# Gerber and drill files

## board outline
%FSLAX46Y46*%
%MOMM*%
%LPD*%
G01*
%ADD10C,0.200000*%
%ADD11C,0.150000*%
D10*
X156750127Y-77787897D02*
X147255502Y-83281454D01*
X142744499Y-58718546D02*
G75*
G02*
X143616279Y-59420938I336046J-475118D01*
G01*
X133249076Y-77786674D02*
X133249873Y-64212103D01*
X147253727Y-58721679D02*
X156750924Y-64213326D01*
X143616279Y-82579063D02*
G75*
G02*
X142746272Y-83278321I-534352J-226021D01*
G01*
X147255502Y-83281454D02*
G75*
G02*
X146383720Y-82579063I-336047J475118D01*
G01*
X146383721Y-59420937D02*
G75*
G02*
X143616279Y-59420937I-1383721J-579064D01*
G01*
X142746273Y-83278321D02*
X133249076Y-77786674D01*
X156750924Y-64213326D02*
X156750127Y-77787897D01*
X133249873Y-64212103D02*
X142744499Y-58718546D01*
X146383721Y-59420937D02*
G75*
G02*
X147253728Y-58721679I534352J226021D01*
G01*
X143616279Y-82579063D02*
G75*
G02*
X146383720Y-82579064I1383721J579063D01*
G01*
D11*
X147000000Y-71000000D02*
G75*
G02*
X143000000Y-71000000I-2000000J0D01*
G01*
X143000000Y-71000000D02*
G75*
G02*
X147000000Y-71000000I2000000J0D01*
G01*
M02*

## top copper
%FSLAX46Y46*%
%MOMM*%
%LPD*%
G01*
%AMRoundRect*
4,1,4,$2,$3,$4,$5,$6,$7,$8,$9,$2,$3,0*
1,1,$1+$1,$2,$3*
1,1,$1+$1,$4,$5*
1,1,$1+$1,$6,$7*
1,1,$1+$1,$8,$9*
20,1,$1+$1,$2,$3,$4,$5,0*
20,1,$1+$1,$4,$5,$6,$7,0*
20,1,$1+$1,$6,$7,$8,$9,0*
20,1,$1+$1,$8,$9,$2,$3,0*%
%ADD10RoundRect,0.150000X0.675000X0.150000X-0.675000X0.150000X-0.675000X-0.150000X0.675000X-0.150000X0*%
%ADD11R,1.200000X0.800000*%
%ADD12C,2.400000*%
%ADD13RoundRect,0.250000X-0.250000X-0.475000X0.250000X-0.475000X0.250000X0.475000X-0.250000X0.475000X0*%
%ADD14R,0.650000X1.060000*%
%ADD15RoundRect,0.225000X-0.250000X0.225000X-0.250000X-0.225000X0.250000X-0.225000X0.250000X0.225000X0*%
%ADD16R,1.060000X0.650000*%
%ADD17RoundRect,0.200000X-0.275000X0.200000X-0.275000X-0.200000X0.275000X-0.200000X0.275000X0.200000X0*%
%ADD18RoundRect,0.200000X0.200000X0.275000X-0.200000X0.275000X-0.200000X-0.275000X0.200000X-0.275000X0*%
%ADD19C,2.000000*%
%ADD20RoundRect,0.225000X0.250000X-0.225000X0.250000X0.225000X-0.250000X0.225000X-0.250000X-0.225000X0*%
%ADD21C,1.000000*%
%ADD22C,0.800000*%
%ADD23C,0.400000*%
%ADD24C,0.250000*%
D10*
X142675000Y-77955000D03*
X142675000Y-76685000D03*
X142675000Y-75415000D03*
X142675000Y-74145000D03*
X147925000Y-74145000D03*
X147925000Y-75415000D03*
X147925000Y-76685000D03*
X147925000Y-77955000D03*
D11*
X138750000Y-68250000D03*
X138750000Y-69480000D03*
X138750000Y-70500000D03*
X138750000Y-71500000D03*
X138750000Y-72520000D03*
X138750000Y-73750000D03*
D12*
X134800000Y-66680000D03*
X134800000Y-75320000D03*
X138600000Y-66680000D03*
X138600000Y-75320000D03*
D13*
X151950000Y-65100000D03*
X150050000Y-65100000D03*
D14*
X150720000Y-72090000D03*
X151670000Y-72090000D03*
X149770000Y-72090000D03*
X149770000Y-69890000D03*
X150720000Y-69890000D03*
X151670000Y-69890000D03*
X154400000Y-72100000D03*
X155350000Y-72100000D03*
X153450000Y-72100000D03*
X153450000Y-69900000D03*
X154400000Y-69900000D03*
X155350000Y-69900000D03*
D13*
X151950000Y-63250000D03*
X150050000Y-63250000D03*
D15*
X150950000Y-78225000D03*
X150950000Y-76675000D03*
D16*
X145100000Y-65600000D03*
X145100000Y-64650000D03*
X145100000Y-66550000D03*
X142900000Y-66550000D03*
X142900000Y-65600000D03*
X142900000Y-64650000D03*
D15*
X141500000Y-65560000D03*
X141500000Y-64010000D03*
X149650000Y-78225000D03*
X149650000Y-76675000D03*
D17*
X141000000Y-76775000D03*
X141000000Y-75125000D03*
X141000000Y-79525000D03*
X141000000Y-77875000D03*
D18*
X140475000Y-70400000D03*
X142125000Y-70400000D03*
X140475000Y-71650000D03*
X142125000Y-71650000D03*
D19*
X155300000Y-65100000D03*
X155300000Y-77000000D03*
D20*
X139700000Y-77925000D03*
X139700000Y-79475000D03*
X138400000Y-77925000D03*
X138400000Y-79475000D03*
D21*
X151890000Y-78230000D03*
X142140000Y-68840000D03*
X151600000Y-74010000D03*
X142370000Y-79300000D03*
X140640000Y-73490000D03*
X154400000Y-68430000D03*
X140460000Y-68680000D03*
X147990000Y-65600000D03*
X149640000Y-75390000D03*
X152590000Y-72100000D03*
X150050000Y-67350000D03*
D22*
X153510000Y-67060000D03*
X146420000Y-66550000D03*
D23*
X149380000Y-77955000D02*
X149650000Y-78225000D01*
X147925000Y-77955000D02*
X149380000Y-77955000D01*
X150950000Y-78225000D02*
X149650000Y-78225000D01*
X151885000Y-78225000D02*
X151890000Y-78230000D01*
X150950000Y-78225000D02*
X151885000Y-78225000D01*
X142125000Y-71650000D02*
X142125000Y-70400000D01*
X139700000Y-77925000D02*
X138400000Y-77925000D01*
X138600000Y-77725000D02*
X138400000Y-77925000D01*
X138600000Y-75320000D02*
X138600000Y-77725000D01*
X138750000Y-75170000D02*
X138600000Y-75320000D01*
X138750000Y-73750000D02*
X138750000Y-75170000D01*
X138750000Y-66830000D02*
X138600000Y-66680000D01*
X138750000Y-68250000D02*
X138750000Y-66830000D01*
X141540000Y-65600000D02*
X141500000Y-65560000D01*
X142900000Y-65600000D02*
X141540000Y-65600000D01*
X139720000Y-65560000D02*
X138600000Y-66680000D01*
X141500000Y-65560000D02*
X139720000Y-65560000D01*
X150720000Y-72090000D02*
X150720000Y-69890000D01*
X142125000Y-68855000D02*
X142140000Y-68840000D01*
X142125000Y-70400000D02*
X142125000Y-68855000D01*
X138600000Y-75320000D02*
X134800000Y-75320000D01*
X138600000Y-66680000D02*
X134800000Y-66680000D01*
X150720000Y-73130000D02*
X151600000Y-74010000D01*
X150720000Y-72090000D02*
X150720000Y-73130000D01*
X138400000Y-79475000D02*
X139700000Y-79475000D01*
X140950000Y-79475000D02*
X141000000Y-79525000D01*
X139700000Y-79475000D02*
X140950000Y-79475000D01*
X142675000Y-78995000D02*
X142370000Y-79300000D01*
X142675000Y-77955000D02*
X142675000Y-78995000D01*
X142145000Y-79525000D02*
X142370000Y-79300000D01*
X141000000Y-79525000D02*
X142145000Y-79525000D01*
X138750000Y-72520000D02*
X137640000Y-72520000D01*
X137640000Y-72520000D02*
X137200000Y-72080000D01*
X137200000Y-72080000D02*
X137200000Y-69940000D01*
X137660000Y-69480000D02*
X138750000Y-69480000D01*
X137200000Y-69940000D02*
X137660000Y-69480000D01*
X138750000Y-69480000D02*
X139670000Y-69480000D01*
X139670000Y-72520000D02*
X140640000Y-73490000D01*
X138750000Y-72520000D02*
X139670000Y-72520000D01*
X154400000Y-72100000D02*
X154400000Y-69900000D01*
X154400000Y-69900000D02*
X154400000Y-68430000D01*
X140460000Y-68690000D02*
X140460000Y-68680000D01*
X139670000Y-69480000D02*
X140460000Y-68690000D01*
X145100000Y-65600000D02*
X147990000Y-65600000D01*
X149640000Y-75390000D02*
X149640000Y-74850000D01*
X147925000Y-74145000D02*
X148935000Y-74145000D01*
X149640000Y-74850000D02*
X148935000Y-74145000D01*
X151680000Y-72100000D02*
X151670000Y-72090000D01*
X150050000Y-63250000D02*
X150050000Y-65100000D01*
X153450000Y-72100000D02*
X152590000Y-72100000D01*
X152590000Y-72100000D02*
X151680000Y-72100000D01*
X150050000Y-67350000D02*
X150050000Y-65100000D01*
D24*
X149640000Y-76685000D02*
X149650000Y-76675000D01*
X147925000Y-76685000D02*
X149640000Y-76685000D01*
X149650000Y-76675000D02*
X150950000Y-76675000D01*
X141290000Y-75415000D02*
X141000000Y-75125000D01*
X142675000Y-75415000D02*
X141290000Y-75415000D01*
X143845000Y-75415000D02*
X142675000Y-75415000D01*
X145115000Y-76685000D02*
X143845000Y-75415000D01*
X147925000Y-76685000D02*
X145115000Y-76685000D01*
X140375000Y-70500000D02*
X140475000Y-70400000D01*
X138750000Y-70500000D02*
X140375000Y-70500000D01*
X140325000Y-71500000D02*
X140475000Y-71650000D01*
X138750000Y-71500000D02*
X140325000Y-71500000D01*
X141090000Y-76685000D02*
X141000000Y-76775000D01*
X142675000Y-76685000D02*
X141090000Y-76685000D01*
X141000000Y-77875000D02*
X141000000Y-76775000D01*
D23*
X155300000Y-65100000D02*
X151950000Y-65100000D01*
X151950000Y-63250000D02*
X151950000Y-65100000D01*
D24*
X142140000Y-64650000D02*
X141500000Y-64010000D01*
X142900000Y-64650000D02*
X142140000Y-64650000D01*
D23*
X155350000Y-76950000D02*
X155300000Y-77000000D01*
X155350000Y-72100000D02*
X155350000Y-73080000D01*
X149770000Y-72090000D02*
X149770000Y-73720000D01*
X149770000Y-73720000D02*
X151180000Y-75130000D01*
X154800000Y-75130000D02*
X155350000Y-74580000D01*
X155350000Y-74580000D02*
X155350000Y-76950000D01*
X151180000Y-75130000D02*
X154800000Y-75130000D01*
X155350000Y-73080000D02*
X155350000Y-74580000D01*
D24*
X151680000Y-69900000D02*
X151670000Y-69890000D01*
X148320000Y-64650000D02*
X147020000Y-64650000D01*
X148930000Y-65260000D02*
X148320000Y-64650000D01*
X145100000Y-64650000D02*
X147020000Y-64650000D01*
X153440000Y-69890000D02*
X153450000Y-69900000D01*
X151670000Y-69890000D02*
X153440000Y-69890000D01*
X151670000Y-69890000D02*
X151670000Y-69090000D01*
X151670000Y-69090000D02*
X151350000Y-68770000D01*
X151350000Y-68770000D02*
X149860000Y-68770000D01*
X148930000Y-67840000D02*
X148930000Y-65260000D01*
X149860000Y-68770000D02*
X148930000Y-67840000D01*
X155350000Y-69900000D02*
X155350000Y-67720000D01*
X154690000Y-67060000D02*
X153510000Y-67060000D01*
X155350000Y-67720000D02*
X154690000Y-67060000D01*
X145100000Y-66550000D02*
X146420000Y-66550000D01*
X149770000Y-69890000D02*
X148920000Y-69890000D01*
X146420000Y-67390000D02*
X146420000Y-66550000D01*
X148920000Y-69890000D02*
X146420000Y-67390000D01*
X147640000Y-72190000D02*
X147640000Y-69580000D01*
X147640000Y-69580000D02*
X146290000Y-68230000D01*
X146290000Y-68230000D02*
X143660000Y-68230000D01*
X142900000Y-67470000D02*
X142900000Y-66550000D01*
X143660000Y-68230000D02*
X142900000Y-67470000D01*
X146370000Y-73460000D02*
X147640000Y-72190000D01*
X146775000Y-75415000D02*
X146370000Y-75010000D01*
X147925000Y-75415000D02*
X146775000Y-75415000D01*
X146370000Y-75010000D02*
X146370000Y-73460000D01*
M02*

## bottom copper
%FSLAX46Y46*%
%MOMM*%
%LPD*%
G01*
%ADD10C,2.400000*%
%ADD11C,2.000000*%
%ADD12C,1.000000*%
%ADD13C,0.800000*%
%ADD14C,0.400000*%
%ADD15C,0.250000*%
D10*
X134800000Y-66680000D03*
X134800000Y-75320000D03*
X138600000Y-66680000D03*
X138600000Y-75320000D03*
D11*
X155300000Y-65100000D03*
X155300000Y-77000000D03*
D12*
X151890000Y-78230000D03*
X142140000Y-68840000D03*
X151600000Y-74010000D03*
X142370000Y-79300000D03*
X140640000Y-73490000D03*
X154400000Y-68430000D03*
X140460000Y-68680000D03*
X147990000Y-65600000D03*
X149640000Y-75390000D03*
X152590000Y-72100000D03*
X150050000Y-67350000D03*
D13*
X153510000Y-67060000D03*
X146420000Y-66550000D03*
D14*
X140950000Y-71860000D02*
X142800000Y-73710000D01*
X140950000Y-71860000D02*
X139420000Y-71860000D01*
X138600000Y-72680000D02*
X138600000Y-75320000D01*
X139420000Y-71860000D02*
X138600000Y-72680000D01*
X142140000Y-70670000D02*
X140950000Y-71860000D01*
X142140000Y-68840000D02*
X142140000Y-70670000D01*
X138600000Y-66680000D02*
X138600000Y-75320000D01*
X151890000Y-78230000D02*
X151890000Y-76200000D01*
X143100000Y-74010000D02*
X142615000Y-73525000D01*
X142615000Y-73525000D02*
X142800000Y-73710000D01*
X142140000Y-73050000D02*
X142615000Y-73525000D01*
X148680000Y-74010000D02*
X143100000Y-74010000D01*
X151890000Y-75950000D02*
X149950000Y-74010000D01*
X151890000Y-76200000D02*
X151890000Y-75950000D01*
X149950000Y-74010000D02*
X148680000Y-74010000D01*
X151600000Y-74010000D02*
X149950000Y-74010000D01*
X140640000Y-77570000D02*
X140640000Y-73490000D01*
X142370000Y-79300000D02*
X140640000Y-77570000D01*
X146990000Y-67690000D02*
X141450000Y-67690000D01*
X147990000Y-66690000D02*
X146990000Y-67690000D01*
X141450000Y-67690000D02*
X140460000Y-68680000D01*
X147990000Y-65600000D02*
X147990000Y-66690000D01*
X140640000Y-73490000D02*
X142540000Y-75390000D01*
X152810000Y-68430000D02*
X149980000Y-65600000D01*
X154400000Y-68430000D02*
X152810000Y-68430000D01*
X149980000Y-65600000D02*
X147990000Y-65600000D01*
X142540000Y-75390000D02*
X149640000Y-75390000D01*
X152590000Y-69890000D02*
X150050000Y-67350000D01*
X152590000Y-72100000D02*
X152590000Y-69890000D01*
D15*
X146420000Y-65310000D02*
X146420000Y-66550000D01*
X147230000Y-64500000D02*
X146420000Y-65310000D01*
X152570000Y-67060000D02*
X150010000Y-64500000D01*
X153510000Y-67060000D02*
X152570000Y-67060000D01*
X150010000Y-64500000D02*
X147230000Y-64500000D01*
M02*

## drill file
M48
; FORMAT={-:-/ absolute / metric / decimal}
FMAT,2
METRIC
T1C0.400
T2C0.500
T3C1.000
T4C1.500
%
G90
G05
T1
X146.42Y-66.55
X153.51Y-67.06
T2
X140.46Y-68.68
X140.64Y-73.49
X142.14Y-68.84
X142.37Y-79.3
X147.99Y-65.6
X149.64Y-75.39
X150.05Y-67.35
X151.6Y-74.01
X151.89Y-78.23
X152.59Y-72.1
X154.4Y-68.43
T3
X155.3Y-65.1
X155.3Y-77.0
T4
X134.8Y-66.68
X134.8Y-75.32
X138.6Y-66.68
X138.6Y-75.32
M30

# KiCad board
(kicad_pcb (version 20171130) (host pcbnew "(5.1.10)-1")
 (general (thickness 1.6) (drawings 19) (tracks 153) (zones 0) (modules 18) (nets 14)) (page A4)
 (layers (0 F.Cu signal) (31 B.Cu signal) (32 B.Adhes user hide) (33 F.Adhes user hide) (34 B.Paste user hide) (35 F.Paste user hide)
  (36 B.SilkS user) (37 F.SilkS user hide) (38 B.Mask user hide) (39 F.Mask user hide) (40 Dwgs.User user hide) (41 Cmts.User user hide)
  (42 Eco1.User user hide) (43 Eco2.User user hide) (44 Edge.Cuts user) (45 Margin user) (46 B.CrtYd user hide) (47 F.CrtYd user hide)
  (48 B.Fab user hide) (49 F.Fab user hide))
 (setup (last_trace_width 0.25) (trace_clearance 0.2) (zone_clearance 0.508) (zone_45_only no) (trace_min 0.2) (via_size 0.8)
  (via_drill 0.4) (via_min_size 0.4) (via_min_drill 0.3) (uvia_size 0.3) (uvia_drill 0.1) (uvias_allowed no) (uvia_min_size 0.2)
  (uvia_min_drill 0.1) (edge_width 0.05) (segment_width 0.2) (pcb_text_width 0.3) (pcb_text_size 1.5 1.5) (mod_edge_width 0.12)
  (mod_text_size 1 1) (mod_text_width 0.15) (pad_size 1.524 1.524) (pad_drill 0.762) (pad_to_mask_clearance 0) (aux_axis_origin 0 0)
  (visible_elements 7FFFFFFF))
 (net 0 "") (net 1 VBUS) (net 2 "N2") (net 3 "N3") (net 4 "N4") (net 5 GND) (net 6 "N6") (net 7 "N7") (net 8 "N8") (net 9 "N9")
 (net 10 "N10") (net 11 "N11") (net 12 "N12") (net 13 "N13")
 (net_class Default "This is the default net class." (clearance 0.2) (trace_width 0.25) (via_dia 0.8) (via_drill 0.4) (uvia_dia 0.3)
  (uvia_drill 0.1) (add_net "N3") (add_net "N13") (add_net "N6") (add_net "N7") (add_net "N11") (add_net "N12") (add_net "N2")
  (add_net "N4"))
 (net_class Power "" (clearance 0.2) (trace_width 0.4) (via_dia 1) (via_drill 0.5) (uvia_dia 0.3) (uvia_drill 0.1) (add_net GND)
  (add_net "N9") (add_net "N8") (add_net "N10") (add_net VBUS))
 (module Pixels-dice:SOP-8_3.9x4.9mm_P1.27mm (layer F.Cu) (at 145.3 76.05 180)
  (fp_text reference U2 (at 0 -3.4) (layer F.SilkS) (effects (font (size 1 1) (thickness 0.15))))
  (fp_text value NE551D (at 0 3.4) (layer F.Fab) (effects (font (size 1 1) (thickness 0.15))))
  (pad 8 smd roundrect (at 2.625 -1.905 180) (size 1.65 0.6) (layers F.Cu F.Paste F.Mask) (roundrect_rratio 0.25) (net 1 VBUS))
  (pad 7 smd roundrect (at 2.625 -0.635 180) (size 1.65 0.6) (layers F.Cu F.Paste F.Mask) (roundrect_rratio 0.25) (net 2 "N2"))
  (pad 6 smd roundrect (at 2.625 0.635 180) (size 1.65 0.6) (layers F.Cu F.Paste F.Mask) (roundrect_rratio 0.25) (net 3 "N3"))
  (pad 5 smd roundrect (at 2.625 1.905 180) (size 1.65 0.6) (layers F.Cu F.Paste F.Mask) (roundrect_rratio 0.25))
  (pad 4 smd roundrect (at -2.625 1.905 180) (size 1.65 0.6) (layers F.Cu F.Paste F.Mask) (roundrect_rratio 0.25) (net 1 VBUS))
  (pad 3 smd roundrect (at -2.625 0.635 180) (size 1.65 0.6) (layers F.Cu F.Paste F.Mask) (roundrect_rratio 0.25) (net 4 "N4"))
  (pad 2 smd roundrect (at -2.625 -0.635 180) (size 1.65 0.6) (layers F.Cu F.Paste F.Mask) (roundrect_rratio 0.25) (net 3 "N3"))
  (pad 1 smd roundrect (at -2.625 -1.905 180) (size 1.65 0.6) (layers F.Cu F.Paste F.Mask) (roundrect_rratio 0.25) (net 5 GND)))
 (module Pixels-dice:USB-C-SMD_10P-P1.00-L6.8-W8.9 (layer F.Cu) (at 136.7 71)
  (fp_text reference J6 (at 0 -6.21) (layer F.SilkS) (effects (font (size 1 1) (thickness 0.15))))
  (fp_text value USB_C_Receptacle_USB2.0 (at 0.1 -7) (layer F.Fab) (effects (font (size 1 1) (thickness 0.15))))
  (pad B12 smd rect (at 2.05 -2.75 270) (size 0.8 1.2) (layers F.Cu F.Paste F.Mask) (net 5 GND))
  (pad B9 smd rect (at 2.05 -1.52 270) (size 0.8 1.2) (layers F.Cu F.Paste F.Mask) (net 1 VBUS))
  (pad A5 smd rect (at 2.05 -0.5 270) (size 0.8 1.2) (layers F.Cu F.Paste F.Mask) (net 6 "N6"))
  (pad B5 smd rect (at 2.05 0.5 270) (size 0.8 1.2) (layers F.Cu F.Paste F.Mask) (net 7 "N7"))
  (pad A9 smd rect (at 2.05 1.52 270) (size 0.8 1.2) (layers F.Cu F.Paste F.Mask) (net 1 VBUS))
  (pad A12 smd rect (at 2.05 2.75 270) (size 0.8 1.2) (layers F.Cu F.Paste F.Mask) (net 5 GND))
  (pad S1 thru_hole circle (at -1.9 -4.32 270) (size 2.4 2.4) (drill 1.5) (layers *.Cu *.Mask) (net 5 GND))
  (pad S1 thru_hole circle (at -1.9 4.32 270) (size 2.4 2.4) (drill 1.5) (layers *.Cu *.Mask) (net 5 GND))
  (pad S1 thru_hole circle (at 1.9 -4.32 270) (size 2.4 2.4) (drill 1.5) (layers *.Cu *.Mask) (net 5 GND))
  (pad S1 thru_hole circle (at 1.9 4.32 270) (size 2.4 2.4) (drill 1.5) (layers *.Cu *.Mask) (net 5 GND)))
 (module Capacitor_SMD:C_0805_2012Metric (layer F.Cu) (at 151 65.1)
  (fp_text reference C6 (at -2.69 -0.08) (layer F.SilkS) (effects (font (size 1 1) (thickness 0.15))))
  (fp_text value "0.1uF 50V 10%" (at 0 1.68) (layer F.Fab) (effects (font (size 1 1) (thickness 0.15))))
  (pad 2 smd roundrect (at 0.95 0) (size 1 1.45) (layers F.Cu F.Paste F.Mask) (roundrect_rratio 0.25) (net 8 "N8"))
  (pad 1 smd roundrect (at -0.95 0) (size 1 1.45) (layers F.Cu F.Paste F.Mask) (roundrect_rratio 0.25) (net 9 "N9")))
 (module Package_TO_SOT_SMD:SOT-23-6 (layer F.Cu) (at 150.72 70.99 270)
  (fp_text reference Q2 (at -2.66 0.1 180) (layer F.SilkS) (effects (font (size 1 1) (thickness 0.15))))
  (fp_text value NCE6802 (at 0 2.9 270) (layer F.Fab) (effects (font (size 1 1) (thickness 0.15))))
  (pad 5 smd rect (at 1.1 0 270) (size 1.06 0.65) (layers F.Cu F.Paste F.Mask) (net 5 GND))
  (pad 6 smd rect (at 1.1 -0.95 270) (size 1.06 0.65) (layers F.Cu F.Paste F.Mask) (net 9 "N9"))
  (pad 4 smd rect (at 1.1 0.95 270) (size 1.06 0.65) (layers F.Cu F.Paste F.Mask) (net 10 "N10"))
  (pad 3 smd rect (at -1.1 0.95 270) (size 1.06 0.65) (layers F.Cu F.Paste F.Mask) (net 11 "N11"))
  (pad 2 smd rect (at -1.1 0 270) (size 1.06 0.65) (layers F.Cu F.Paste F.Mask) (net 5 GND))
  (pad 1 smd rect (at -1.1 -0.95 270) (size 1.06 0.65) (layers F.Cu F.Paste F.Mask) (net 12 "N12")))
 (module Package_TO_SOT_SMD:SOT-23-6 (layer F.Cu) (at 154.4 71 270)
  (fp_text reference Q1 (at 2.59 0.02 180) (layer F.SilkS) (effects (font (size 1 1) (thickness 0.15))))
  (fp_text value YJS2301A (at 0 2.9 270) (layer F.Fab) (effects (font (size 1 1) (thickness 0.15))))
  (pad 5 smd rect (at 1.1 0 270) (size 1.06 0.65) (layers F.Cu F.Paste F.Mask) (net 1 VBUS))
  (pad 6 smd rect (at 1.1 -0.95 270) (size 1.06 0.65) (layers F.Cu F.Paste F.Mask) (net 10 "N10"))
  (pad 4 smd rect (at 1.1 0.95 270) (size 1.06 0.65) (layers F.Cu F.Paste F.Mask) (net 9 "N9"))
  (pad 3 smd rect (at -1.1 0.95 270) (size 1.06 0.65) (layers F.Cu F.Paste F.Mask) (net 12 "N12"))
  (pad 2 smd rect (at -1.1 0 270) (size 1.06 0.65) (layers F.Cu F.Paste F.Mask) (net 1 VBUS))
  (pad 1 smd rect (at -1.1 -0.95 270) (size 1.06 0.65) (layers F.Cu F.Paste F.Mask) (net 11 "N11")))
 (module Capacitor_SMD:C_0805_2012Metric (layer F.Cu) (at 151 63.25)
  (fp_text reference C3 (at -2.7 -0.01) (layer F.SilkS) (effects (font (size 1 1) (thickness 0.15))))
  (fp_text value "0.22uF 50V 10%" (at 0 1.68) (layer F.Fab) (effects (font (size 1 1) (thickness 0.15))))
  (pad 2 smd roundrect (at 0.95 0) (size 1 1.45) (layers F.Cu F.Paste F.Mask) (roundrect_rratio 0.25) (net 8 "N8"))
  (pad 1 smd roundrect (at -0.95 0) (size 1 1.45) (layers F.Cu F.Paste F.Mask) (roundrect_rratio 0.25) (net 9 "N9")))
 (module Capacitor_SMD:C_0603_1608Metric (layer F.Cu) (at 150.95 77.45 270)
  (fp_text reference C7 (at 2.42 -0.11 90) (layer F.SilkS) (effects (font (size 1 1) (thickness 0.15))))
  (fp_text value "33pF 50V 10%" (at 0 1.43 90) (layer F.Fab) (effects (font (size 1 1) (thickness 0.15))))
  (pad 2 smd roundrect (at 0.775 0 270) (size 0.9 0.95) (layers F.Cu F.Paste F.Mask) (roundrect_rratio 0.25) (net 5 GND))
  (pad 1 smd roundrect (at -0.775 0 270) (size 0.9 0.95) (layers F.Cu F.Paste F.Mask) (roundrect_rratio 0.25) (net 3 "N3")))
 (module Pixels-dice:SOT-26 (layer F.Cu) (at 144 65.6 180)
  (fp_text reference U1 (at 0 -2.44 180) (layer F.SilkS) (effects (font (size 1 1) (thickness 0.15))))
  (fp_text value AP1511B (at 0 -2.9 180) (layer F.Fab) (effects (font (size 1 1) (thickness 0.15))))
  (pad 5 smd rect (at -1.1 0) (size 1.06 0.65) (layers F.Cu F.Paste F.Mask) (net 1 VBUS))
  (pad 6 smd rect (at -1.1 0.95) (size 1.06 0.65) (layers F.Cu F.Paste F.Mask) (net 12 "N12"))
  (pad 4 smd rect (at -1.1 -0.95) (size 1.06 0.65) (layers F.Cu F.Paste F.Mask) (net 11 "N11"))
  (pad 3 smd rect (at 1.1 -0.95) (size 1.06 0.65) (layers F.Cu F.Paste F.Mask) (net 4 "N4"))
  (pad 2 smd rect (at 1.1 0) (size 1.06 0.65) (layers F.Cu F.Paste F.Mask) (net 5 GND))
  (pad 1 smd rect (at 1.1 0.95) (size 1.06 0.65) (layers F.Cu F.Paste F.Mask) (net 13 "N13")))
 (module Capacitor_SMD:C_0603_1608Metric (layer F.Cu) (at 141.5 64.785 270)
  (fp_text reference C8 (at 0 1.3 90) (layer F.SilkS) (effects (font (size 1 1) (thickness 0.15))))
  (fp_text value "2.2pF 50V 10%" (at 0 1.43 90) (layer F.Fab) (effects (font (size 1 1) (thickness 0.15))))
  (pad 2 smd roundrect (at 0.775 0 270) (size 0.9 0.95) (layers F.Cu F.Paste F.Mask) (roundrect_rratio 0.25) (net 5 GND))
  (pad 1 smd roundrect (at -0.775 0 270) (size 0.9 0.95) (layers F.Cu F.Paste F.Mask) (roundrect_rratio 0.25) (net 13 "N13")))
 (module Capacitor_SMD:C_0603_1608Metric (layer F.Cu) (at 149.65 77.45 270)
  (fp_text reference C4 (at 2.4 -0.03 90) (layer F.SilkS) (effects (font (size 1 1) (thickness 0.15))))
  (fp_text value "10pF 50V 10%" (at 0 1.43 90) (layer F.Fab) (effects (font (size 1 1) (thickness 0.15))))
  (pad 2 smd roundrect (at 0.775 0 270) (size 0.9 0.95) (layers F.Cu F.Paste F.Mask) (roundrect_rratio 0.25) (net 5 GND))
  (pad 1 smd roundrect (at -0.775 0 270) (size 0.9 0.95) (layers F.Cu F.Paste F.Mask) (roundrect_rratio 0.25) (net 3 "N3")))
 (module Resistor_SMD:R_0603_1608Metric (layer F.Cu) (at 141 75.95 270)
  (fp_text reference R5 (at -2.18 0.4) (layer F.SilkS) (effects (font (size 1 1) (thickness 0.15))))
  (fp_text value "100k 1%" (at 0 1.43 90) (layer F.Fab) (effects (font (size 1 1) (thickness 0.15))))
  (pad 2 smd roundrect (at 0.825 0 270) (size 0.8 0.95) (layers F.Cu F.Paste F.Mask) (roundrect_rratio 0.25) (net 2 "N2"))
  (pad 1 smd roundrect (at -0.825 0 270) (size 0.8 0.95) (layers F.Cu F.Paste F.Mask) (roundrect_rratio 0.25) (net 3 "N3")))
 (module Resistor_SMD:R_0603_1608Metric (layer F.Cu) (at 141 78.7 270)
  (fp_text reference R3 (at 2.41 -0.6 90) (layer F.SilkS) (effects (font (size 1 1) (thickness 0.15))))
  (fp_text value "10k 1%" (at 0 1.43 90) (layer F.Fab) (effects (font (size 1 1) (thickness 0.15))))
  (pad 2 smd roundrect (at 0.825 0 270) (size 0.8 0.95) (layers F.Cu F.Paste F.Mask) (roundrect_rratio 0.25) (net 1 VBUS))
  (pad 1 smd roundrect (at -0.825 0 270) (size 0.8 0.95) (layers F.Cu F.Paste F.Mask) (roundrect_rratio 0.25) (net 2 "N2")))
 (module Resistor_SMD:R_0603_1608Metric (layer F.Cu) (at 141.3 70.4 180)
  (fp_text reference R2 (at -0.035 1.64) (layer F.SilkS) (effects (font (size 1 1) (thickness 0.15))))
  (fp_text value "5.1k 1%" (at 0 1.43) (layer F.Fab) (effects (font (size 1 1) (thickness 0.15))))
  (pad 2 smd roundrect (at 0.825 0 180) (size 0.8 0.95) (layers F.Cu F.Paste F.Mask) (roundrect_rratio 0.25) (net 6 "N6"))
  (pad 1 smd roundrect (at -0.825 0 180) (size 0.8 0.95) (layers F.Cu F.Paste F.Mask) (roundrect_rratio 0.25) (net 5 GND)))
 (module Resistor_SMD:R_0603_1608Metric (layer F.Cu) (at 141.3 71.65 180)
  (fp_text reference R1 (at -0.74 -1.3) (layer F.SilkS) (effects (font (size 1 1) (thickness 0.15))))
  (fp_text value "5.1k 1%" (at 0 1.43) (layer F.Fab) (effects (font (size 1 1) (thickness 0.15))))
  (pad 2 smd roundrect (at 0.825 0 180) (size 0.8 0.95) (layers F.Cu F.Paste F.Mask) (roundrect_rratio 0.25) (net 7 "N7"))
  (pad 1 smd roundrect (at -0.825 0 180) (size 0.8 0.95) (layers F.Cu F.Paste F.Mask) (roundrect_rratio 0.25) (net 5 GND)))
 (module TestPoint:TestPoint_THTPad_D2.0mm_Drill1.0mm (layer F.Cu) (at 155.3 65.1)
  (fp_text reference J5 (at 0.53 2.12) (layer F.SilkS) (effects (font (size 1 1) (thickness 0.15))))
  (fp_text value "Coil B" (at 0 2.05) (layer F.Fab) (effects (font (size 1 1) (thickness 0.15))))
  (pad 1 thru_hole circle (at 0 0) (size 2 2) (drill 1) (layers *.Cu *.Mask) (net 8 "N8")))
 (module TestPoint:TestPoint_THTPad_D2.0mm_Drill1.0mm (layer F.Cu) (at 155.3 77)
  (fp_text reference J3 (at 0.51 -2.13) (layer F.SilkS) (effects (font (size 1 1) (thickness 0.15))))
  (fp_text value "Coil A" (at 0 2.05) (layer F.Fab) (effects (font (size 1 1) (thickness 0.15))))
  (pad 1 thru_hole circle (at 0 0) (size 2 2) (drill 1) (layers *.Cu *.Mask) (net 10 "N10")))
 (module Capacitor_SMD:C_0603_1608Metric (layer F.Cu) (at 139.7 78.7 90)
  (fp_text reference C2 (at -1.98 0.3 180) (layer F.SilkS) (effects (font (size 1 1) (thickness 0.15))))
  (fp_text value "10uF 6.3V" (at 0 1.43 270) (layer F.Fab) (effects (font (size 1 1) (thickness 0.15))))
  (pad 2 smd roundrect (at 0.775 0 90) (size 0.9 0.95) (layers F.Cu F.Paste F.Mask) (roundrect_rratio 0.25) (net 5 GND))
  (pad 1 smd roundrect (at -0.775 0 90) (size 0.9 0.95) (layers F.Cu F.Paste F.Mask) (roundrect_rratio 0.25) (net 1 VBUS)))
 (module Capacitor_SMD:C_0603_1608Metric (layer F.Cu) (at 138.4 78.7 90)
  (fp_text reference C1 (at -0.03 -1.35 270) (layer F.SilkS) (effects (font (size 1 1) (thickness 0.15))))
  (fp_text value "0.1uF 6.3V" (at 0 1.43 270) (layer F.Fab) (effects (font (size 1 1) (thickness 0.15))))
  (pad 2 smd roundrect (at 0.775 0 90) (size 0.9 0.95) (layers F.Cu F.Paste F.Mask) (roundrect_rratio 0.25) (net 5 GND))
  (pad 1 smd roundrect (at -0.775 0 90) (size 0.9 0.95) (layers F.Cu F.Paste F.Mask) (roundrect_rratio 0.25) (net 1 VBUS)))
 (gr_line (start 156.750127 77.787897) (end 147.255502 83.281454) (layer Edge.Cuts) (width 0.2))
 (gr_arc (start 143.080545 59.193664) (end 142.744499 58.718546) (angle 148.2594298) (layer Edge.Cuts) (width 0.2))
 (gr_line (start 133.249076 77.786674) (end 133.249873 64.212103) (layer Edge.Cuts) (width 0.2))
 (gr_line (start 147.253727 58.721679) (end 156.750924 64.213326) (layer Edge.Cuts) (width 0.2))
 (gr_arc (start 143.081927 82.805084) (end 143.616279 82.579063) (angle 148.274571) (layer Edge.Cuts) (width 0.2))
 (gr_arc (start 146.919455 82.806336) (end 147.255502 83.281454) (angle 148.2594298) (layer Edge.Cuts) (width 0.2))
 (gr_arc (start 145 60.000001) (end 146.383721 59.420937) (angle 225.4169665) (layer Edge.Cuts) (width 0.2))
 (gr_line (start 142.746273 83.278321) (end 133.249076 77.786674) (layer Edge.Cuts) (width 0.2))
 (gr_line (start 156.750924 64.213326) (end 156.750127 77.787897) (layer Edge.Cuts) (width 0.2))
 (gr_line (start 133.249873 64.212103) (end 142.744499 58.718546) (layer Edge.Cuts) (width 0.2))
 (gr_arc (start 146.918073 59.194916) (end 146.383721 59.420937) (angle 148.274571) (layer Edge.Cuts) (width 0.2))
 (gr_arc (start 145 82) (end 143.616279 82.579063) (angle 225.4169665) (layer Edge.Cuts) (width 0.2))
 (gr_circle (center 145 71) (end 147 71) (layer Edge.Cuts) (width 0.15))
 (segment (start 149.38 77.955) (end 149.65 78.225) (width 0.4) (layer F.Cu) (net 5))
 (segment (start 147.925 77.955) (end 149.38 77.955) (width 0.4) (layer F.Cu) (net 5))
 (segment (start 150.95 78.225) (end 149.65 78.225) (width 0.4) (layer F.Cu) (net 5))
 (via (at 151.89 78.23) (size 1) (drill 0.5) (layers F.Cu B.Cu) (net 5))
 (segment (start 151.885 78.225) (end 151.89 78.23) (width 0.4) (layer F.Cu) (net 5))
 (segment (start 150.95 78.225) (end 151.885 78.225) (width 0.4) (layer F.Cu) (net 5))
 (segment (start 142.125 71.65) (end 142.125 70.4) (width 0.4) (layer F.Cu) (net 5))
 (via (at 142.14 68.84) (size 1) (drill 0.5) (layers F.Cu B.Cu) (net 5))
 (segment (start 139.7 77.925) (end 138.4 77.925) (width 0.4) (layer F.Cu) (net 5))
 (segment (start 138.6 77.725) (end 138.4 77.925) (width 0.4) (layer F.Cu) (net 5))
 (segment (start 138.6 75.32) (end 138.6 77.725) (width 0.4) (layer F.Cu) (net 5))
 (segment (start 138.75 75.17) (end 138.6 75.32) (width 0.4) (layer F.Cu) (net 5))
 (segment (start 138.75 73.75) (end 138.75 75.17) (width 0.4) (layer F.Cu) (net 5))
 (segment (start 138.75 66.83) (end 138.6 66.68) (width 0.4) (layer F.Cu) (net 5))
 (segment (start 138.75 68.25) (end 138.75 66.83) (width 0.4) (layer F.Cu) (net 5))
 (segment (start 141.54 65.6) (end 141.5 65.56) (width 0.4) (layer F.Cu) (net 5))
 (segment (start 142.9 65.6) (end 141.54 65.6) (width 0.4) (layer F.Cu) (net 5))
 (segment (start 139.72 65.56) (end 138.6 66.68) (width 0.4) (layer F.Cu) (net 5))
 (segment (start 141.5 65.56) (end 139.72 65.56) (width 0.4) (layer F.Cu) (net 5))
 (segment (start 150.72 72.09) (end 150.72 69.89) (width 0.4) (layer F.Cu) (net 5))
 (segment (start 140.95 71.86) (end 142.8 73.71) (width 0.4) (layer B.Cu) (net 5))
 (segment (start 140.95 71.86) (end 139.42 71.86) (width 0.4) (layer B.Cu) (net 5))
 (segment (start 138.6 72.68) (end 138.6 75.32) (width 0.4) (layer B.Cu) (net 5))
 (segment (start 139.42 71.86) (end 138.6 72.68) (width 0.4) (layer B.Cu) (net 5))
 (segment (start 142.125 68.855) (end 142.14 68.84) (width 0.4) (layer F.Cu) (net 5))
 (segment (start 142.125 70.4) (end 142.125 68.855) (width 0.4) (layer F.Cu) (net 5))
 (segment (start 138.6 75.32) (end 134.8 75.32) (width 0.4) (layer F.Cu) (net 5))
 (segment (start 138.6 66.68) (end 134.8 66.68) (width 0.4) (layer F.Cu) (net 5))
 (segment (start 142.14 70.67) (end 140.95 71.86) (width 0.4) (layer B.Cu) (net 5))
 (segment (start 142.14 68.84) (end 142.14 70.67) (width 0.4) (layer B.Cu) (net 5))
 (segment (start 138.6 66.68) (end 138.6 75.32) (width 0.4) (layer B.Cu) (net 5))
 (segment (start 151.89 78.23) (end 151.89 76.2) (width 0.4) (layer B.Cu) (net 5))
 (via (at 151.6 74.01) (size 1) (drill 0.5) (layers F.Cu B.Cu) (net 5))
 (segment (start 150.72 73.13) (end 151.6 74.01) (width 0.4) (layer F.Cu) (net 5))
 (segment (start 150.72 72.09) (end 150.72 73.13) (width 0.4) (layer F.Cu) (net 5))
 (segment (start 143.1 74.01) (end 142.615 73.525) (width 0.4) (layer B.Cu) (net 5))
 (segment (start 142.615 73.525) (end 142.8 73.71) (width 0.4) (layer B.Cu) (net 5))
 (segment (start 142.14 73.05) (end 142.615 73.525) (width 0.4) (layer B.Cu) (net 5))
 (segment (start 148.68 74.01) (end 143.1 74.01) (width 0.4) (layer B.Cu) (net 5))
 (segment (start 151.89 75.95) (end 149.95 74.01) (width 0.4) (layer B.Cu) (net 5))
 (segment (start 151.89 76.2) (end 151.89 75.95) (width 0.4) (layer B.Cu) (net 5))
 (segment (start 149.95 74.01) (end 148.68 74.01) (width 0.4) (layer B.Cu) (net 5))
 (segment (start 151.6 74.01) (end 149.95 74.01) (width 0.4) (layer B.Cu) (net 5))
 (segment (start 138.4 79.475) (end 139.7 79.475) (width 0.4) (layer F.Cu) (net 1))
 (segment (start 140.95 79.475) (end 141 79.525) (width 0.4) (layer F.Cu) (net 1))
 (segment (start 139.7 79.475) (end 140.95 79.475) (width 0.4) (layer F.Cu) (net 1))
 (segment (start 142.675 78.995) (end 142.37 79.3) (width 0.4) (layer F.Cu) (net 1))
 (via (at 142.37 79.3) (size 1) (drill 0.5) (layers F.Cu B.Cu) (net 1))
 (segment (start 142.675 77.955) (end 142.675 78.995) (width 0.4) (layer F.Cu) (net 1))
 (segment (start 142.145 79.525) (end 142.37 79.3) (width 0.4) (layer F.Cu) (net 1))
 (segment (start 141 79.525) (end 142.145 79.525) (width 0.4) (layer F.Cu) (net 1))
 (segment (start 138.75 72.52) (end 137.64 72.52) (width 0.4) (layer F.Cu) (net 1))
 (segment (start 137.64 72.52) (end 137.2 72.08) (width 0.4) (layer F.Cu) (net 1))
 (segment (start 137.2 72.08) (end 137.2 69.94) (width 0.4) (layer F.Cu) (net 1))
 (segment (start 137.66 69.48) (end 138.75 69.48) (width 0.4) (layer F.Cu) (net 1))
 (segment (start 137.2 69.94) (end 137.66 69.48) (width 0.4) (layer F.Cu) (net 1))
 (segment (start 138.75 69.48) (end 139.67 69.48) (width 0.4) (layer F.Cu) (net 1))
 (via (at 140.64 73.49) (size 1) (drill 0.5) (layers F.Cu B.Cu) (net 1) (status 1000000))
 (segment (start 139.67 72.52) (end 140.64 73.49) (width 0.4) (layer F.Cu) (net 1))
 (segment (start 138.75 72.52) (end 139.67 72.52) (width 0.4) (layer F.Cu) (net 1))
 (segment (start 154.4 72.1) (end 154.4 69.9) (width 0.4) (layer F.Cu) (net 1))
 (via (at 154.4 68.43) (size 1) (drill 0.5) (layers F.Cu B.Cu) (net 1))
 (segment (start 154.4 69.9) (end 154.4 68.43) (width 0.4) (layer F.Cu) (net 1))
 (segment (start 140.64 77.57) (end 140.64 73.49) (width 0.4) (layer B.Cu) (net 1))
 (segment (start 142.37 79.3) (end 140.64 77.57) (width 0.4) (layer B.Cu) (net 1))
 (segment (start 140.46 68.69) (end 140.46 68.68) (width 0.4) (layer F.Cu) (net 1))
 (via (at 140.46 68.68) (size 1) (drill 0.5) (layers F.Cu B.Cu) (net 1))
 (segment (start 139.67 69.48) (end 140.46 68.69) (width 0.4) (layer F.Cu) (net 1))
 (segment (start 145.1 65.6) (end 147.99 65.6) (width 0.4) (layer F.Cu) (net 1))
 (via (at 147.99 65.6) (size 1) (drill 0.5) (layers F.Cu B.Cu) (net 1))
 (segment (start 146.99 67.69) (end 141.45 67.69) (width 0.4) (layer B.Cu) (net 1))
 (segment (start 147.99 66.69) (end 146.99 67.69) (width 0.4) (layer B.Cu) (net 1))
 (segment (start 141.45 67.69) (end 140.46 68.68) (width 0.4) (layer B.Cu) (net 1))
 (segment (start 147.99 65.6) (end 147.99 66.69) (width 0.4) (layer B.Cu) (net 1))
 (segment (start 140.64 73.49) (end 142.54 75.39) (width 0.4) (layer B.Cu) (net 1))
 (segment (start 152.81 68.43) (end 149.98 65.6) (width 0.4) (layer B.Cu) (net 1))
 (segment (start 154.4 68.43) (end 152.81 68.43) (width 0.4) (layer B.Cu) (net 1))
 (segment (start 149.98 65.6) (end 147.99 65.6) (width 0.4) (layer B.Cu) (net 1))
 (via (at 149.64 75.39) (size 1) (drill 0.5) (layers F.Cu B.Cu) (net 1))
 (segment (start 149.64 75.39) (end 149.64 74.85) (width 0.4) (layer F.Cu) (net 1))
 (segment (start 147.925 74.145) (end 148.935 74.145) (width 0.4) (layer F.Cu) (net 1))
 (segment (start 149.64 74.85) (end 148.935 74.145) (width 0.4) (layer F.Cu) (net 1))
 (segment (start 142.54 75.39) (end 149.64 75.39) (width 0.4) (layer B.Cu) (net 1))
 (segment (start 151.68 72.1) (end 151.67 72.09) (width 0.4) (layer F.Cu) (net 9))
 (segment (start 150.05 63.25) (end 150.05 65.1) (width 0.4) (layer F.Cu) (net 9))
 (segment (start 153.45 72.1) (end 152.59 72.1) (width 0.4) (layer F.Cu) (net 9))
 (segment (start 152.59 72.1) (end 151.68 72.1) (width 0.4) (layer F.Cu) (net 9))
 (via (at 152.59 72.1) (size 1) (drill 0.5) (layers F.Cu B.Cu) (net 9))
 (via (at 150.05 67.35) (size 1) (drill 0.5) (layers F.Cu B.Cu) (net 9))
 (segment (start 150.05 67.35) (end 150.05 65.1) (width 0.4) (layer F.Cu) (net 9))
 (segment (start 152.59 69.89) (end 150.05 67.35) (width 0.4) (layer B.Cu) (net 9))
 (segment (start 152.59 72.1) (end 152.59 69.89) (width 0.4) (layer B.Cu) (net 9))
 (segment (start 149.64 76.685) (end 149.65 76.675) (width 0.25) (layer F.Cu) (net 3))
 (segment (start 147.925 76.685) (end 149.64 76.685) (width 0.25) (layer F.Cu) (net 3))
 (segment (start 149.65 76.675) (end 150.95 76.675) (width 0.25) (layer F.Cu) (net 3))
 (segment (start 141.29 75.415) (end 141 75.125) (width 0.25) (layer F.Cu) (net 3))
 (segment (start 142.675 75.415) (end 141.29 75.415) (width 0.25) (layer F.Cu) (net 3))
 (segment (start 143.845 75.415) (end 142.675 75.415) (width 0.25) (layer F.Cu) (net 3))
 (segment (start 145.115 76.685) (end 143.845 75.415) (width 0.25) (layer F.Cu) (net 3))
 (segment (start 147.925 76.685) (end 145.115 76.685) (width 0.25) (layer F.Cu) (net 3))
 (segment (start 140.375 70.5) (end 140.475 70.4) (width 0.25) (layer F.Cu) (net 6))
 (segment (start 138.75 70.5) (end 140.375 70.5) (width 0.25) (layer F.Cu) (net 6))
 (segment (start 140.325 71.5) (end 140.475 71.65) (width 0.25) (layer F.Cu) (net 7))
 (segment (start 138.75 71.5) (end 140.325 71.5) (width 0.25) (layer F.Cu) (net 7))
 (segment (start 141.09 76.685) (end 141 76.775) (width 0.25) (layer F.Cu) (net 2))
 (segment (start 142.675 76.685) (end 141.09 76.685) (width 0.25) (layer F.Cu) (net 2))
 (segment (start 141 77.875) (end 141 76.775) (width 0.25) (layer F.Cu) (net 2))
 (segment (start 155.3 65.1) (end 151.95 65.1) (width 0.4) (layer F.Cu) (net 8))
 (segment (start 151.95 63.25) (end 151.95 65.1) (width 0.4) (layer F.Cu) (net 8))
 (segment (start 142.14 64.65) (end 141.5 64.01) (width 0.25) (layer F.Cu) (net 13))
 (segment (start 142.9 64.65) (end 142.14 64.65) (width 0.25) (layer F.Cu) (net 13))
 (segment (start 155.35 76.95) (end 155.3 77) (width 0.4) (layer F.Cu) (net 10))
 (segment (start 155.35 72.1) (end 155.35 73.08) (width 0.4) (layer F.Cu) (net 10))
 (segment (start 149.77 72.09) (end 149.77 73.72) (width 0.4) (layer F.Cu) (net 10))
 (segment (start 149.77 73.72) (end 151.18 75.13) (width 0.4) (layer F.Cu) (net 10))
 (segment (start 154.8 75.13) (end 155.35 74.58) (width 0.4) (layer F.Cu) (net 10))
 (segment (start 155.35 74.58) (end 155.35 76.95) (width 0.4) (layer F.Cu) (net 10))
 (segment (start 151.18 75.13) (end 154.8 75.13) (width 0.4) (layer F.Cu) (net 10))
 (segment (start 155.35 73.08) (end 155.35 74.58) (width 0.4) (layer F.Cu) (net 10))
 (segment (start 151.68 69.9) (end 151.67 69.89) (width 0.25) (layer F.Cu) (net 12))
 (segment (start 148.32 64.65) (end 147.02 64.65) (width 0.25) (layer F.Cu) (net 12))
 (segment (start 148.93 65.26) (end 148.32 64.65) (width 0.25) (layer F.Cu) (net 12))
 (segment (start 145.1 64.65) (end 147.02 64.65) (width 0.25) (layer F.Cu) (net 12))
 (segment (start 153.44 69.89) (end 153.45 69.9) (width 0.25) (layer F.Cu) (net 12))
 (segment (start 151.67 69.89) (end 153.44 69.89) (width 0.25) (layer F.Cu) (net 12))
 (segment (start 151.67 69.89) (end 151.67 69.09) (width 0.25) (layer F.Cu) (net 12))
 (segment (start 151.67 69.09) (end 151.35 68.77) (width 0.25) (layer F.Cu) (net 12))
 (segment (start 151.35 68.77) (end 149.86 68.77) (width 0.25) (layer F.Cu) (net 12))
 (segment (start 148.93 67.84) (end 148.93 65.26) (width 0.25) (layer F.Cu) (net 12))
 (segment (start 149.86 68.77) (end 148.93 67.84) (width 0.25) (layer F.Cu) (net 12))
 (segment (start 155.35 69.9) (end 155.35 67.72) (width 0.25) (layer F.Cu) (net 11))
 (segment (start 154.69 67.06) (end 153.51 67.06) (width 0.25) (layer F.Cu) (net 11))
 (via (at 153.51 67.06) (size 0.8) (drill 0.4) (layers F.Cu B.Cu) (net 11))
 (segment (start 155.35 67.72) (end 154.69 67.06) (width 0.25) (layer F.Cu) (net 11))
 (via (at 146.42 66.55) (size 0.8) (drill 0.4) (layers F.Cu B.Cu) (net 11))
 (segment (start 145.1 66.55) (end 146.42 66.55) (width 0.25) (layer F.Cu) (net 11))
 (segment (start 146.42 65.31) (end 146.42 66.55) (width 0.25) (layer B.Cu) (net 11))
 (segment (start 147.23 64.5) (end 146.42 65.31) (width 0.25) (layer B.Cu) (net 11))
 (segment (start 149.77 69.89) (end 148.92 69.89) (width 0.25) (layer F.Cu) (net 11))
 (segment (start 146.42 67.39) (end 146.42 66.55) (width 0.25) (layer F.Cu) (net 11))
 (segment (start 148.92 69.89) (end 146.42 67.39) (width 0.25) (layer F.Cu) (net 11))
 (segment (start 152.57 67.06) (end 150.01 64.5) (width 0.25) (layer B.Cu) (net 11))
 (segment (start 153.51 67.06) (end 152.57 67.06) (width 0.25) (layer B.Cu) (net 11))
 (segment (start 150.01 64.5) (end 147.23 64.5) (width 0.25) (layer B.Cu) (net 11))
 (segment (start 147.64 72.19) (end 147.64 69.58) (width 0.25) (layer F.Cu) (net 4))
 (segment (start 147.64 69.58) (end 146.29 68.23) (width 0.25) (layer F.Cu) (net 4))
 (segment (start 146.29 68.23) (end 143.66 68.23) (width 0.25) (layer F.Cu) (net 4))
 (segment (start 142.9 67.47) (end 142.9 66.55) (width 0.25) (layer F.Cu) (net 4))
 (segment (start 143.66 68.23) (end 142.9 67.47) (width 0.25) (layer F.Cu) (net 4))
 (segment (start 146.37 73.46) (end 147.64 72.19) (width 0.25) (layer F.Cu) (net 4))
 (segment (start 146.775 75.415) (end 146.37 75.01) (width 0.25) (layer F.Cu) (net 4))
 (segment (start 147.925 75.415) (end 146.775 75.415) (width 0.25) (layer F.Cu) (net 4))
 (segment (start 146.37 75.01) (end 146.37 73.46) (width 0.25) (layer F.Cu) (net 4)))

